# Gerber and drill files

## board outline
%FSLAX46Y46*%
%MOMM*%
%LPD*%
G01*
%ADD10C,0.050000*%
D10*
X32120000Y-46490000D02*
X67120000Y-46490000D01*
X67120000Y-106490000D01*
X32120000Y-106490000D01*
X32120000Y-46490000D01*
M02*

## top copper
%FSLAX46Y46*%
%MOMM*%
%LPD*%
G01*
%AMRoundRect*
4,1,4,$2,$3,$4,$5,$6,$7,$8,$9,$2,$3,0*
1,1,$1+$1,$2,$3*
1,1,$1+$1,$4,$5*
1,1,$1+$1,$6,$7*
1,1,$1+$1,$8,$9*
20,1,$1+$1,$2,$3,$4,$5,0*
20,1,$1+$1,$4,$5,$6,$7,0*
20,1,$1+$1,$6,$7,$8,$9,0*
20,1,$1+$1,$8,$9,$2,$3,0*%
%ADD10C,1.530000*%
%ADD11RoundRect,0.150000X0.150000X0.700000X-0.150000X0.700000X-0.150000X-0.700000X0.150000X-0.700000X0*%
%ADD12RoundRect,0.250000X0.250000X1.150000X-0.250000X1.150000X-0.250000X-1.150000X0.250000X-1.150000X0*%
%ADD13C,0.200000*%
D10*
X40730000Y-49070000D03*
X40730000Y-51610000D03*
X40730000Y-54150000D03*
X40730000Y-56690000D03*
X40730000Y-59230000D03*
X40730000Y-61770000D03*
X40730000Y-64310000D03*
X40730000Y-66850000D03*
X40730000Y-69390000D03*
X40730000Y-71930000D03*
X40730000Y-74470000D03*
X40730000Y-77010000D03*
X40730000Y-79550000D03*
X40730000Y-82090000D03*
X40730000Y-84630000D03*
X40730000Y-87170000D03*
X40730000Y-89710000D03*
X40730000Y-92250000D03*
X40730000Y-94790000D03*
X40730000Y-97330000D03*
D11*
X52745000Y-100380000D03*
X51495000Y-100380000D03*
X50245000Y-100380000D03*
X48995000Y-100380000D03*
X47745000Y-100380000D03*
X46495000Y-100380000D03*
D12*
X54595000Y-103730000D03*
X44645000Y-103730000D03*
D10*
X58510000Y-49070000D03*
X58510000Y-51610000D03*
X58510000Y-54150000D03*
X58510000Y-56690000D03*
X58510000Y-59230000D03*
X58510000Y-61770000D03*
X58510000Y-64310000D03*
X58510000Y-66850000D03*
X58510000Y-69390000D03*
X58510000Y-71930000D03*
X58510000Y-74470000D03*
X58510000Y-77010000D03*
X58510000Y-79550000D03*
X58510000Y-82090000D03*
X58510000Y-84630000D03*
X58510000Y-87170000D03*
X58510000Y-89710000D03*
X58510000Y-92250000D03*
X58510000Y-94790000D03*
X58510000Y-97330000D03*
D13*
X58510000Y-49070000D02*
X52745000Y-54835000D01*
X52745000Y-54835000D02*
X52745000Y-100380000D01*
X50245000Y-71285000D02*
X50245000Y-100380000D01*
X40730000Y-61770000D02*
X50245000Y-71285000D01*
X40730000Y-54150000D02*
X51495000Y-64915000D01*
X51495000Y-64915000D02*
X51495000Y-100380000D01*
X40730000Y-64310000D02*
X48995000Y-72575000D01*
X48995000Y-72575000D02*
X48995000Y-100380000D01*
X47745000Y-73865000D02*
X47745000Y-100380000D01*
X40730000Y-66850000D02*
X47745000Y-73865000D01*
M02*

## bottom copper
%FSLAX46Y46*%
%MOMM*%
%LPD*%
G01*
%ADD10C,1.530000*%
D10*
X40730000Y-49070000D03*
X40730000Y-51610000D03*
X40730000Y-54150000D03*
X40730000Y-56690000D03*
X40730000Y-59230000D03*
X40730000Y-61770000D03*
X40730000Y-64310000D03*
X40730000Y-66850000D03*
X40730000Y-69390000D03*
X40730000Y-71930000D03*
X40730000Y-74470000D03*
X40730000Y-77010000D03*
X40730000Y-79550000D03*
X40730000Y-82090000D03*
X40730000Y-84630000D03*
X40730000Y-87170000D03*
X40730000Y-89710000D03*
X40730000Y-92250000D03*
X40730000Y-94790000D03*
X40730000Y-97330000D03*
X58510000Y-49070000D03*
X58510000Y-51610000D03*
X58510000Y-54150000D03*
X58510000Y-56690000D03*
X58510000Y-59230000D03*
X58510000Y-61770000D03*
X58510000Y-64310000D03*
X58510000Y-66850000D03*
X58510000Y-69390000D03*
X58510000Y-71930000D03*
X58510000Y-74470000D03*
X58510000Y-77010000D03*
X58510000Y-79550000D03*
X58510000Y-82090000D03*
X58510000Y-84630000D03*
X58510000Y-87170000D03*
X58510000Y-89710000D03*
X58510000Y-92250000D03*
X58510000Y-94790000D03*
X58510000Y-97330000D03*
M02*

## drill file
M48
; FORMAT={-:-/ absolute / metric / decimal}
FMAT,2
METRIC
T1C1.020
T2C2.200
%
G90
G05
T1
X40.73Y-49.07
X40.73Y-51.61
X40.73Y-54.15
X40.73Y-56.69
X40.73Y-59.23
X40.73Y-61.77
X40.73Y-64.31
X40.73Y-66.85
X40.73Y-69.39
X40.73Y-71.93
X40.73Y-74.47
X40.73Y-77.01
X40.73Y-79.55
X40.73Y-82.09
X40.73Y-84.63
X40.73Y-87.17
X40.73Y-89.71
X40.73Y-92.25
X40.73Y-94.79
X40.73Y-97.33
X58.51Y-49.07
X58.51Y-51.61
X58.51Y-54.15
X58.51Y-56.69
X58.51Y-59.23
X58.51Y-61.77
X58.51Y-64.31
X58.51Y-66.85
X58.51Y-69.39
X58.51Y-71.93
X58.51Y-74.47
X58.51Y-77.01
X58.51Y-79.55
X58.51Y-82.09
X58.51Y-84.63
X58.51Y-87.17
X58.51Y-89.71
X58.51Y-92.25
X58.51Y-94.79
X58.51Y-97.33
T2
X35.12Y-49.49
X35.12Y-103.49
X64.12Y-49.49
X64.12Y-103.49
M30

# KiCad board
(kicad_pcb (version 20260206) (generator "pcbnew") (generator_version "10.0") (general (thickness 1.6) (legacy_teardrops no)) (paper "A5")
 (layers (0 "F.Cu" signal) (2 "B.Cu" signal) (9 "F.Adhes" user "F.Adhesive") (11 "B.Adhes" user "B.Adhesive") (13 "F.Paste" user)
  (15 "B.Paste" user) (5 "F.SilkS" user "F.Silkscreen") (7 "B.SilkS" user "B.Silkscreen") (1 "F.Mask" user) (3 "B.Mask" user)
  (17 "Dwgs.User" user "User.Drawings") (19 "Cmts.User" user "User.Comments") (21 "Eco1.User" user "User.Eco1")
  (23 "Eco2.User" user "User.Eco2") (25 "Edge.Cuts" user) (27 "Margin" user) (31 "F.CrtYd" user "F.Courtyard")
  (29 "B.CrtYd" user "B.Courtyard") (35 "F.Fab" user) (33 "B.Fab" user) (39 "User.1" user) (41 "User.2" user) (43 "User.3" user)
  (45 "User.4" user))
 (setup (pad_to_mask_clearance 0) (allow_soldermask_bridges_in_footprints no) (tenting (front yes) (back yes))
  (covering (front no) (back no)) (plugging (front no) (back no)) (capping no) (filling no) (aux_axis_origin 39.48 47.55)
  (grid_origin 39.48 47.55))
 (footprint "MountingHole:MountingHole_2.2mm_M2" (layer "F.Cu") (at 35.12 49.49)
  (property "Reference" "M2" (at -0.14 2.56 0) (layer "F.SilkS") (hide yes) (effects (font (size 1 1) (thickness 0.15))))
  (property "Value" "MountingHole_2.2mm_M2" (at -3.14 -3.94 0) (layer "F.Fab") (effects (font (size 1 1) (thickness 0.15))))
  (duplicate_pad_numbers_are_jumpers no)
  (pad "" np_thru_hole circle (at 0 0) (size 2.2 2.2) (drill 2.2) (layers "*.Cu" "*.Mask")))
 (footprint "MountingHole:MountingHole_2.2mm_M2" (layer "F.Cu") (at 64.12 49.49)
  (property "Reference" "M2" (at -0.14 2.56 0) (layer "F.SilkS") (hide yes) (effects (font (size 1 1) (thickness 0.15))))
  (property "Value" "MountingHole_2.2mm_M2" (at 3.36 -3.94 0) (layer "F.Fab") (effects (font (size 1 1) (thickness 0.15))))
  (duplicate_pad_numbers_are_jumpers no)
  (pad "" np_thru_hole circle (at 0 0) (size 2.2 2.2) (drill 2.2) (layers "*.Cu" "*.Mask")))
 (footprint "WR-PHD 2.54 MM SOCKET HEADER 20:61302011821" (layer "F.Cu") (at 40.73 73.2 -90)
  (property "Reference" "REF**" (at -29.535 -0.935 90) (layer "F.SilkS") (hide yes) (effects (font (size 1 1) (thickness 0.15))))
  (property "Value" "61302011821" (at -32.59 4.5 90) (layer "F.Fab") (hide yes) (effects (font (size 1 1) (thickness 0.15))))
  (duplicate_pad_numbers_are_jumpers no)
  (pad "1" thru_hole circle (at -24.13 0 270) (size 1.53 1.53) (drill 1.02) (layers "*.Cu" "*.Mask") (remove_unused_layers no)
   (solder_mask_margin 0.102))
  (pad "2" thru_hole circle (at -21.59 0 270) (size 1.53 1.53) (drill 1.02) (layers "*.Cu" "*.Mask") (remove_unused_layers no)
   (solder_mask_margin 0.102))
  (pad "3" thru_hole circle (at -19.05 0 270) (size 1.53 1.53) (drill 1.02) (layers "*.Cu" "*.Mask") (remove_unused_layers no) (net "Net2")
   (solder_mask_margin 0.102))
  (pad "4" thru_hole circle (at -16.51 0 270) (size 1.53 1.53) (drill 1.02) (layers "*.Cu" "*.Mask") (remove_unused_layers no)
   (solder_mask_margin 0.102))
  (pad "5" thru_hole circle (at -13.97 0 270) (size 1.53 1.53) (drill 1.02) (layers "*.Cu" "*.Mask") (remove_unused_layers no)
   (solder_mask_margin 0.102))
  (pad "6" thru_hole circle (at -11.43 0 270) (size 1.53 1.53) (drill 1.02) (layers "*.Cu" "*.Mask") (remove_unused_layers no) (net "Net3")
   (solder_mask_margin 0.102))
  (pad "7" thru_hole circle (at -8.89 0 270) (size 1.53 1.53) (drill 1.02) (layers "*.Cu" "*.Mask") (remove_unused_layers no) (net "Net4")
   (solder_mask_margin 0.102))
  (pad "8" thru_hole circle (at -6.35 0 270) (size 1.53 1.53) (drill 1.02) (layers "*.Cu" "*.Mask") (remove_unused_layers no) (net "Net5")
   (solder_mask_margin 0.102))
  (pad "9" thru_hole circle (at -3.81 0 270) (size 1.53 1.53) (drill 1.02) (layers "*.Cu" "*.Mask") (remove_unused_layers no)
   (solder_mask_margin 0.102))
  (pad "10" thru_hole circle (at -1.27 0 270) (size 1.53 1.53) (drill 1.02) (layers "*.Cu" "*.Mask") (remove_unused_layers no)
   (solder_mask_margin 0.102))
  (pad "11" thru_hole circle (at 1.27 0 270) (size 1.53 1.53) (drill 1.02) (layers "*.Cu" "*.Mask") (remove_unused_layers no)
   (solder_mask_margin 0.102))
  (pad "12" thru_hole circle (at 3.81 0 270) (size 1.53 1.53) (drill 1.02) (layers "*.Cu" "*.Mask") (remove_unused_layers no)
   (solder_mask_margin 0.102))
  (pad "13" thru_hole circle (at 6.35 0 270) (size 1.53 1.53) (drill 1.02) (layers "*.Cu" "*.Mask") (remove_unused_layers no)
   (solder_mask_margin 0.102))
  (pad "14" thru_hole circle (at 8.89 0 270) (size 1.53 1.53) (drill 1.02) (layers "*.Cu" "*.Mask") (remove_unused_layers no)
   (solder_mask_margin 0.102))
  (pad "15" thru_hole circle (at 11.43 0 270) (size 1.53 1.53) (drill 1.02) (layers "*.Cu" "*.Mask") (remove_unused_layers no)
   (solder_mask_margin 0.102))
  (pad "16" thru_hole circle (at 13.97 0 270) (size 1.53 1.53) (drill 1.02) (layers "*.Cu" "*.Mask") (remove_unused_layers no)
   (solder_mask_margin 0.102))
  (pad "17" thru_hole circle (at 16.51 0 270) (size 1.53 1.53) (drill 1.02) (layers "*.Cu" "*.Mask") (remove_unused_layers no)
   (solder_mask_margin 0.102))
  (pad "18" thru_hole circle (at 19.05 0 270) (size 1.53 1.53) (drill 1.02) (layers "*.Cu" "*.Mask") (remove_unused_layers no)
   (solder_mask_margin 0.102))
  (pad "19" thru_hole circle (at 21.59 0 270) (size 1.53 1.53) (drill 1.02) (layers "*.Cu" "*.Mask") (remove_unused_layers no)
   (solder_mask_margin 0.102))
  (pad "20" thru_hole circle (at 24.13 0 270) (size 1.53 1.53) (drill 1.02) (layers "*.Cu" "*.Mask") (remove_unused_layers no)
   (solder_mask_margin 0.102)))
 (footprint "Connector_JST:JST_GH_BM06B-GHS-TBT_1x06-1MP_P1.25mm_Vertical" (layer "F.Cu") (at 49.62 102.33 180)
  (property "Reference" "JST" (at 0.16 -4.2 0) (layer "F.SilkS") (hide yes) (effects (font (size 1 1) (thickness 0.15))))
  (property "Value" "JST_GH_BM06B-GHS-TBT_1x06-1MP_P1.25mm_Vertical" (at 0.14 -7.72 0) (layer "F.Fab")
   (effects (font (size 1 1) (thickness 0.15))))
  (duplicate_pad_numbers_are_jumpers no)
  (pad "1" smd roundrect (at -3.125 1.95 180) (size 0.6 1.7) (layers "F.Cu" "F.Mask" "F.Paste") (roundrect_rratio 0.25) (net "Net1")
   (solder_mask_margin 0))
  (pad "2" smd roundrect (at -1.875 1.95 180) (size 0.6 1.7) (layers "F.Cu" "F.Mask" "F.Paste") (roundrect_rratio 0.25) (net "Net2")
   (solder_mask_margin 0))
  (pad "3" smd roundrect (at -0.625 1.95 180) (size 0.6 1.7) (layers "F.Cu" "F.Mask" "F.Paste") (roundrect_rratio 0.25) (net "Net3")
   (solder_mask_margin 0))
  (pad "4" smd roundrect (at 0.625 1.95 180) (size 0.6 1.7) (layers "F.Cu" "F.Mask" "F.Paste") (roundrect_rratio 0.25) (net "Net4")
   (solder_mask_margin 0))
  (pad "5" smd roundrect (at 1.875 1.95 180) (size 0.6 1.7) (layers "F.Cu" "F.Mask" "F.Paste") (roundrect_rratio 0.25) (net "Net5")
   (solder_mask_margin 0))
  (pad "6" smd roundrect (at 3.125 1.95 180) (size 0.6 1.7) (layers "F.Cu" "F.Mask" "F.Paste") (roundrect_rratio 0.25))
  (pad "MP" smd roundrect (at -4.975 -1.4 180) (size 1 2.8) (layers "F.Cu" "F.Mask" "F.Paste") (roundrect_rratio 0.25))
  (pad "MP" smd roundrect (at 4.975 -1.4 180) (size 1 2.8) (layers "F.Cu" "F.Mask" "F.Paste") (roundrect_rratio 0.25)))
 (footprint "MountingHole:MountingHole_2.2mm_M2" (layer "F.Cu") (at 35.12 103.49)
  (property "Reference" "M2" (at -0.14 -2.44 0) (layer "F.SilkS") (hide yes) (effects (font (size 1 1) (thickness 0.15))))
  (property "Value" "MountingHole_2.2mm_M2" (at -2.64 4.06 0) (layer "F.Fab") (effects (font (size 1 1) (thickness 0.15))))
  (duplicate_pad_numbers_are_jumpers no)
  (pad "" np_thru_hole circle (at 0 0) (size 2.2 2.2) (drill 2.2) (layers "*.Cu" "*.Mask")))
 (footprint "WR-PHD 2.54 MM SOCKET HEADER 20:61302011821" (layer "F.Cu") (at 58.51 73.2 -90)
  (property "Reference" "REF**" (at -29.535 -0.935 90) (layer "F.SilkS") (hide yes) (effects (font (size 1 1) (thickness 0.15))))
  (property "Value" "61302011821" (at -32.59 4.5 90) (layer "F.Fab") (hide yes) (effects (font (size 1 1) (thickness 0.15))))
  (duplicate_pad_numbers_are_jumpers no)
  (pad "1" thru_hole circle (at -24.13 0 270) (size 1.53 1.53) (drill 1.02) (layers "*.Cu" "*.Mask") (remove_unused_layers no) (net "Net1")
   (solder_mask_margin 0.102))
  (pad "2" thru_hole circle (at -21.59 0 270) (size 1.53 1.53) (drill 1.02) (layers "*.Cu" "*.Mask") (remove_unused_layers no)
   (solder_mask_margin 0.102))
  (pad "3" thru_hole circle (at -19.05 0 270) (size 1.53 1.53) (drill 1.02) (layers "*.Cu" "*.Mask") (remove_unused_layers no)
   (solder_mask_margin 0.102))
  (pad "4" thru_hole circle (at -16.51 0 270) (size 1.53 1.53) (drill 1.02) (layers "*.Cu" "*.Mask") (remove_unused_layers no)
   (solder_mask_margin 0.102))
  (pad "5" thru_hole circle (at -13.97 0 270) (size 1.53 1.53) (drill 1.02) (layers "*.Cu" "*.Mask") (remove_unused_layers no)
   (solder_mask_margin 0.102))
  (pad "6" thru_hole circle (at -11.43 0 270) (size 1.53 1.53) (drill 1.02) (layers "*.Cu" "*.Mask") (remove_unused_layers no)
   (solder_mask_margin 0.102))
  (pad "7" thru_hole circle (at -8.89 0 270) (size 1.53 1.53) (drill 1.02) (layers "*.Cu" "*.Mask") (remove_unused_layers no)
   (solder_mask_margin 0.102))
  (pad "8" thru_hole circle (at -6.35 0 270) (size 1.53 1.53) (drill 1.02) (layers "*.Cu" "*.Mask") (remove_unused_layers no)
   (solder_mask_margin 0.102))
  (pad "9" thru_hole circle (at -3.81 0 270) (size 1.53 1.53) (drill 1.02) (layers "*.Cu" "*.Mask") (remove_unused_layers no)
   (solder_mask_margin 0.102))
  (pad "10" thru_hole circle (at -1.27 0 270) (size 1.53 1.53) (drill 1.02) (layers "*.Cu" "*.Mask") (remove_unused_layers no)
   (solder_mask_margin 0.102))
  (pad "11" thru_hole circle (at 1.27 0 270) (size 1.53 1.53) (drill 1.02) (layers "*.Cu" "*.Mask") (remove_unused_layers no)
   (solder_mask_margin 0.102))
  (pad "12" thru_hole circle (at 3.81 0 270) (size 1.53 1.53) (drill 1.02) (layers "*.Cu" "*.Mask") (remove_unused_layers no)
   (solder_mask_margin 0.102))
  (pad "13" thru_hole circle (at 6.35 0 270) (size 1.53 1.53) (drill 1.02) (layers "*.Cu" "*.Mask") (remove_unused_layers no)
   (solder_mask_margin 0.102))
  (pad "14" thru_hole circle (at 8.89 0 270) (size 1.53 1.53) (drill 1.02) (layers "*.Cu" "*.Mask") (remove_unused_layers no)
   (solder_mask_margin 0.102))
  (pad "15" thru_hole circle (at 11.43 0 270) (size 1.53 1.53) (drill 1.02) (layers "*.Cu" "*.Mask") (remove_unused_layers no)
   (solder_mask_margin 0.102))
  (pad "16" thru_hole circle (at 13.97 0 270) (size 1.53 1.53) (drill 1.02) (layers "*.Cu" "*.Mask") (remove_unused_layers no)
   (solder_mask_margin 0.102))
  (pad "17" thru_hole circle (at 16.51 0 270) (size 1.53 1.53) (drill 1.02) (layers "*.Cu" "*.Mask") (remove_unused_layers no)
   (solder_mask_margin 0.102))
  (pad "18" thru_hole circle (at 19.05 0 270) (size 1.53 1.53) (drill 1.02) (layers "*.Cu" "*.Mask") (remove_unused_layers no)
   (solder_mask_margin 0.102))
  (pad "19" thru_hole circle (at 21.59 0 270) (size 1.53 1.53) (drill 1.02) (layers "*.Cu" "*.Mask") (remove_unused_layers no)
   (solder_mask_margin 0.102))
  (pad "20" thru_hole circle (at 24.13 0 270) (size 1.53 1.53) (drill 1.02) (layers "*.Cu" "*.Mask") (remove_unused_layers no)
   (solder_mask_margin 0.102)))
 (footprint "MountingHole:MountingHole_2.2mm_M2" (layer "F.Cu") (at 64.12 103.49)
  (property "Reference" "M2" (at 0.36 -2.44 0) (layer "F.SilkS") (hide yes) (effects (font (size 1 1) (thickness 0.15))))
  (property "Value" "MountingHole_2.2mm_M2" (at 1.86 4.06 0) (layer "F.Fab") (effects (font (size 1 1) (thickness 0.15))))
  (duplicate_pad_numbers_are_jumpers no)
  (pad "" np_thru_hole circle (at 0 0) (size 2.2 2.2) (drill 2.2) (layers "*.Cu" "*.Mask")))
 (gr_rect (start 32.12 46.49) (end 67.12 106.49) (stroke (width 0.05) (type solid)) (fill no) (layer "Edge.Cuts"))
 (segment (start 58.51 49.07) (end 52.745 54.835) (width 0.2) (layer "F.Cu") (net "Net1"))
 (segment (start 52.745 54.835) (end 52.745 100.38) (width 0.2) (layer "F.Cu") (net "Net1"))
 (segment (start 50.245 71.285) (end 50.245 100.38) (width 0.2) (layer "F.Cu") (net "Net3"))
 (segment (start 40.73 61.77) (end 50.245 71.285) (width 0.2) (layer "F.Cu") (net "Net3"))
 (segment (start 40.73 54.15) (end 51.495 64.915) (width 0.2) (layer "F.Cu") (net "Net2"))
 (segment (start 51.495 64.915) (end 51.495 100.38) (width 0.2) (layer "F.Cu") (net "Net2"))
 (segment (start 40.73 64.31) (end 48.995 72.575) (width 0.2) (layer "F.Cu") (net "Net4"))
 (segment (start 48.995 72.575) (end 48.995 100.38) (width 0.2) (layer "F.Cu") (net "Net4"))
 (segment (start 47.745 73.865) (end 47.745 100.38) (width 0.2) (layer "F.Cu") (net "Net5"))
 (segment (start 40.73 66.85) (end 47.745 73.865) (width 0.2) (layer "F.Cu") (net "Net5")))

